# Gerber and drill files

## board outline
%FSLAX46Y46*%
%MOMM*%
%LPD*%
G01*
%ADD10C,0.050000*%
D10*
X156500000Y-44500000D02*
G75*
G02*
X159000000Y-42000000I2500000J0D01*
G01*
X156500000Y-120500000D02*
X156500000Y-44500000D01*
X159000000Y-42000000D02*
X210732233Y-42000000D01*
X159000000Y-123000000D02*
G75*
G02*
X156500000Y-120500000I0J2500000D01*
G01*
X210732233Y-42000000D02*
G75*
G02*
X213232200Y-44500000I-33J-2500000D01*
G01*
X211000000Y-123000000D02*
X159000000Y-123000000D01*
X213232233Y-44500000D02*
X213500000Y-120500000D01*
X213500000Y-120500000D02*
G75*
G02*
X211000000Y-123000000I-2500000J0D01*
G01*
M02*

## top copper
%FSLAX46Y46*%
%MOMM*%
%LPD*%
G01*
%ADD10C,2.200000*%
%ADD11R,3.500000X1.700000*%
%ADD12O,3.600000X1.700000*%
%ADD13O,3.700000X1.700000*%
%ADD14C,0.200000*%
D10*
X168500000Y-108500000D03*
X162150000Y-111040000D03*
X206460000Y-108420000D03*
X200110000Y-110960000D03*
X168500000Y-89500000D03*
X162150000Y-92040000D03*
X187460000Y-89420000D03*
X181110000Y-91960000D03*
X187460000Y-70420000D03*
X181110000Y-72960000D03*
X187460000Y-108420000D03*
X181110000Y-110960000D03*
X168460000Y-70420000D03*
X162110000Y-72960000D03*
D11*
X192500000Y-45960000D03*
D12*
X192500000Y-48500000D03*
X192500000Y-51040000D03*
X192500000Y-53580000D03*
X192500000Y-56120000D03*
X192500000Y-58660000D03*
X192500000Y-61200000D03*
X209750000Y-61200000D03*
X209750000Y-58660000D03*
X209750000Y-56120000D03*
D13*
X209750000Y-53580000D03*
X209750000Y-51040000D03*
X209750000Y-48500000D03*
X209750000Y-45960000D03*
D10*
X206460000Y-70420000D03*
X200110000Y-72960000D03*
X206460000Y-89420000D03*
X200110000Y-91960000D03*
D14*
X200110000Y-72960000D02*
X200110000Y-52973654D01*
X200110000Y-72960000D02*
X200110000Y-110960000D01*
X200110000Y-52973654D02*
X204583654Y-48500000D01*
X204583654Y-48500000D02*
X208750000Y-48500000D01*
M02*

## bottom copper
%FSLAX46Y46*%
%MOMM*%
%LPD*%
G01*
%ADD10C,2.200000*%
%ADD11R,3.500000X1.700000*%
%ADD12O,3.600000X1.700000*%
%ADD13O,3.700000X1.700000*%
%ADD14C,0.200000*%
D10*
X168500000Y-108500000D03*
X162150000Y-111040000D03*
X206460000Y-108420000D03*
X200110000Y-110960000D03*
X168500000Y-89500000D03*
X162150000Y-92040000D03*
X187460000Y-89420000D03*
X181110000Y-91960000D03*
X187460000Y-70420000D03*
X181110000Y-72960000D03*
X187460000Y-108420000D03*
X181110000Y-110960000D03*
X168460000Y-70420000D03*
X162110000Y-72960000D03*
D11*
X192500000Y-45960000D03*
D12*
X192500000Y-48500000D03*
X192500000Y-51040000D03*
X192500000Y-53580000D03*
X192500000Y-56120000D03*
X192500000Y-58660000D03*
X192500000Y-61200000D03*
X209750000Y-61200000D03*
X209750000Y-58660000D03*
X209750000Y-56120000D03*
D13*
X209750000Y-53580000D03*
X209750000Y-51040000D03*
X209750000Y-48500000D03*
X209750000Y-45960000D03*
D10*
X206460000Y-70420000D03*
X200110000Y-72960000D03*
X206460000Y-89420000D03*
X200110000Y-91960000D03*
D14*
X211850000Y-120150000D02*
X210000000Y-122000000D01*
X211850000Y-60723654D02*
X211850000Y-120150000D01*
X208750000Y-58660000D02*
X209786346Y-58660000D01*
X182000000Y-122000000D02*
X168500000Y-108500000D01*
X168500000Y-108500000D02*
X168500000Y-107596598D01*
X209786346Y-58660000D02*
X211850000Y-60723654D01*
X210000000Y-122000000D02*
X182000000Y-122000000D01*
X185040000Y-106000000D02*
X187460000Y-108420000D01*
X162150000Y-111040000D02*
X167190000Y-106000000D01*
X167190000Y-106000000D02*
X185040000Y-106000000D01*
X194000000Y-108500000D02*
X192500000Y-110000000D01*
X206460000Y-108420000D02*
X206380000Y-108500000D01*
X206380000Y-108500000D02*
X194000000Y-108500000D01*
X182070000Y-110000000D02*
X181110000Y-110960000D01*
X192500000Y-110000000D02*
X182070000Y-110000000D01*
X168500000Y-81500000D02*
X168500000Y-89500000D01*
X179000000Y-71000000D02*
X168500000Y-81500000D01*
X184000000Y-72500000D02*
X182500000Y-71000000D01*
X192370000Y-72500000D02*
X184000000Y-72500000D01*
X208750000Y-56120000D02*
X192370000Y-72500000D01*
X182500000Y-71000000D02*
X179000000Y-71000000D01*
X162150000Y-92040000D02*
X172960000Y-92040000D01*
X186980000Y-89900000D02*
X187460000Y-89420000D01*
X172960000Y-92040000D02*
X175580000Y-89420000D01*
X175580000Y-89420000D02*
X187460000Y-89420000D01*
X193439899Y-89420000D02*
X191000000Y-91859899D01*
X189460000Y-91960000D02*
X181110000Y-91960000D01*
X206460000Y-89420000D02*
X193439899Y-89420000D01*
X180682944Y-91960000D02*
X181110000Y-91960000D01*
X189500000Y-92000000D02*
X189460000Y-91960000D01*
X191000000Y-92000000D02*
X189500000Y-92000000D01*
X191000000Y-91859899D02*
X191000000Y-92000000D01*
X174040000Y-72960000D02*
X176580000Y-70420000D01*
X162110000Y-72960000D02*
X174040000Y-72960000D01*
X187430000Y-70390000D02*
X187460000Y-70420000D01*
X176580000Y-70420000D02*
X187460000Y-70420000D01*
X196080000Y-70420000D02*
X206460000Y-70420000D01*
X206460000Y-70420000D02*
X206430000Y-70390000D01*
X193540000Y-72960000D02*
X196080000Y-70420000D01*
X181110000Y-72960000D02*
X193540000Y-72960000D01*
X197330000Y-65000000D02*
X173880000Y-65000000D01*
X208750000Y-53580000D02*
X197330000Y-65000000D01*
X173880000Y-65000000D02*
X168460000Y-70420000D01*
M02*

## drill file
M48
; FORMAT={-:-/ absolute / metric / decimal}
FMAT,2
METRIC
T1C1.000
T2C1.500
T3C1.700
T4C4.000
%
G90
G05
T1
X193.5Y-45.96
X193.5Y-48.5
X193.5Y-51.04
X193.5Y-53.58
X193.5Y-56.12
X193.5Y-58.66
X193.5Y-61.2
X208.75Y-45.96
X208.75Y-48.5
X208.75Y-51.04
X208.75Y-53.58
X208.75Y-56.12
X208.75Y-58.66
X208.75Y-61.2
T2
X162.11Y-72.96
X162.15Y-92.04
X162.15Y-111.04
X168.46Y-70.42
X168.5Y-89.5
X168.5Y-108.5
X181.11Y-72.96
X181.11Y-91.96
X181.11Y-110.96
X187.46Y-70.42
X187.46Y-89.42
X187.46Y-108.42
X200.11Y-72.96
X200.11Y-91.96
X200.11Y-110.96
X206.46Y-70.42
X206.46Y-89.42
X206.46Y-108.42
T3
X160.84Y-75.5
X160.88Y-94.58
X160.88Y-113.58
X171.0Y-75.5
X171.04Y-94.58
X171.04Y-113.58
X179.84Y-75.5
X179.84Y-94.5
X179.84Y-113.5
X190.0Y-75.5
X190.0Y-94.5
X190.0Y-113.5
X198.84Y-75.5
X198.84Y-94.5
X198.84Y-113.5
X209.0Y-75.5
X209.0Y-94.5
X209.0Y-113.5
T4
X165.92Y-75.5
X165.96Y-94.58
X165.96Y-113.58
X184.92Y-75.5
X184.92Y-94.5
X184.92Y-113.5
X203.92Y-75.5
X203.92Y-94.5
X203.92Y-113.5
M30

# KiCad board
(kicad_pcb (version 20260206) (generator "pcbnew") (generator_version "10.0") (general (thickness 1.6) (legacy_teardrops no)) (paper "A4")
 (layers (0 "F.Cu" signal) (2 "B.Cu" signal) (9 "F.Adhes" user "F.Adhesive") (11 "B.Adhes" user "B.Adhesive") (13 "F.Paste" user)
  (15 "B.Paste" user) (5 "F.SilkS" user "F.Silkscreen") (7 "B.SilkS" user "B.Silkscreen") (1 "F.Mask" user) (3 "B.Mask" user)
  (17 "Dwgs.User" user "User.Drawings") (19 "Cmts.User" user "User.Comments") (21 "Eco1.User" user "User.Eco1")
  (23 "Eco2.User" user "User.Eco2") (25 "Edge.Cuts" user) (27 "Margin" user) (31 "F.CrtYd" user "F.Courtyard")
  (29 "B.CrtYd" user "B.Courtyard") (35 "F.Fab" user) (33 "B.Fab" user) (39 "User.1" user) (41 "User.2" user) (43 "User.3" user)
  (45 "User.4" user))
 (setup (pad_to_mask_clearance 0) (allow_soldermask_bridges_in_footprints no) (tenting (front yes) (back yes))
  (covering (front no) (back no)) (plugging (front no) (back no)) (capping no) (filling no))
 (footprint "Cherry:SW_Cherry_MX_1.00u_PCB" (layer "F.Cu") (at 168.5 108.5)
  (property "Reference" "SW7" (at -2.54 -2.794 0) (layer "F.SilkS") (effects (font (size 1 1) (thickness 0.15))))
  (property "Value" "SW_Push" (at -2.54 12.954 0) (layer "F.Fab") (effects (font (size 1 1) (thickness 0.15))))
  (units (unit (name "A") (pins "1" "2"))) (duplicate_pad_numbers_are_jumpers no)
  (pad "" np_thru_hole circle (at -7.62 5.08) (size 1.7 1.7) (drill 1.7) (layers "*.Cu" "*.Mask"))
  (pad "" np_thru_hole circle (at -2.54 5.08) (size 4 4) (drill 4) (layers "*.Cu" "*.Mask"))
  (pad "" np_thru_hole circle (at 2.54 5.08) (size 1.7 1.7) (drill 1.7) (layers "*.Cu" "*.Mask"))
  (pad "1" thru_hole circle (at 0 0) (size 2.2 2.2) (drill 1.5) (layers "*.Cu" "*.Mask") (remove_unused_layers no)
   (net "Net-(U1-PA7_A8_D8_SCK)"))
  (pad "2" thru_hole circle (at -6.35 2.54) (size 2.2 2.2) (drill 1.5) (layers "*.Cu" "*.Mask") (remove_unused_layers no)
   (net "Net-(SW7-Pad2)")))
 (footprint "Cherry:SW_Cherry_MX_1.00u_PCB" (layer "F.Cu") (at 206.46 108.42)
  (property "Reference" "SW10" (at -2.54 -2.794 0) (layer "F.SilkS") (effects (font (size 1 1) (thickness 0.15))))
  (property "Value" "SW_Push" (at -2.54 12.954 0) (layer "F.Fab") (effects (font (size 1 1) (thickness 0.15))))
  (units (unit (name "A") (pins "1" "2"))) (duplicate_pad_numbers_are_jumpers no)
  (pad "" np_thru_hole circle (at -7.62 5.08) (size 1.7 1.7) (drill 1.7) (layers "*.Cu" "*.Mask"))
  (pad "" np_thru_hole circle (at -2.54 5.08) (size 4 4) (drill 4) (layers "*.Cu" "*.Mask"))
  (pad "" np_thru_hole circle (at 2.54 5.08) (size 1.7 1.7) (drill 1.7) (layers "*.Cu" "*.Mask"))
  (pad "1" thru_hole circle (at 0 0) (size 2.2 2.2) (drill 1.5) (layers "*.Cu" "*.Mask") (remove_unused_layers no) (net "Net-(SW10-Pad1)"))
  (pad "2" thru_hole circle (at -6.35 2.54) (size 2.2 2.2) (drill 1.5) (layers "*.Cu" "*.Mask") (remove_unused_layers no) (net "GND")))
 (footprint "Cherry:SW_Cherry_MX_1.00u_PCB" (layer "F.Cu") (at 168.5 89.5)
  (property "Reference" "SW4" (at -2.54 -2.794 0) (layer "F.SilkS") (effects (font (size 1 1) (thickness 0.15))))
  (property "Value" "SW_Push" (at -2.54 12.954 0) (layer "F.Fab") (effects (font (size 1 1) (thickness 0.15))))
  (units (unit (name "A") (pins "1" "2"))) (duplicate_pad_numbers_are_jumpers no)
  (pad "" np_thru_hole circle (at -7.62 5.08) (size 1.7 1.7) (drill 1.7) (layers "*.Cu" "*.Mask"))
  (pad "" np_thru_hole circle (at -2.54 5.08) (size 4 4) (drill 4) (layers "*.Cu" "*.Mask"))
  (pad "" np_thru_hole circle (at 2.54 5.08) (size 1.7 1.7) (drill 1.7) (layers "*.Cu" "*.Mask"))
  (pad "1" thru_hole circle (at 0 0) (size 2.2 2.2) (drill 1.5) (layers "*.Cu" "*.Mask") (remove_unused_layers no)
   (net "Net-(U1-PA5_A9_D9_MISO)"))
  (pad "2" thru_hole circle (at -6.35 2.54) (size 2.2 2.2) (drill 1.5) (layers "*.Cu" "*.Mask") (remove_unused_layers no)
   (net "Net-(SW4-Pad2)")))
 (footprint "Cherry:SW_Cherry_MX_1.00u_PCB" (layer "F.Cu") (at 187.46 89.42)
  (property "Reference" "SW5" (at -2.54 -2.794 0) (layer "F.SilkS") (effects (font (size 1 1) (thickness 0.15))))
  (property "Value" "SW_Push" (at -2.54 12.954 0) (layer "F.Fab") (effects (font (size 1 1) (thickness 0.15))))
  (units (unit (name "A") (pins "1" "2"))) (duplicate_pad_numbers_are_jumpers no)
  (pad "" np_thru_hole circle (at -7.62 5.08) (size 1.7 1.7) (drill 1.7) (layers "*.Cu" "*.Mask"))
  (pad "" np_thru_hole circle (at -2.54 5.08) (size 4 4) (drill 4) (layers "*.Cu" "*.Mask"))
  (pad "" np_thru_hole circle (at 2.54 5.08) (size 1.7 1.7) (drill 1.7) (layers "*.Cu" "*.Mask"))
  (pad "1" thru_hole circle (at 0 0) (size 2.2 2.2) (drill 1.5) (layers "*.Cu" "*.Mask") (remove_unused_layers no) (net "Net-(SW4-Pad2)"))
  (pad "2" thru_hole circle (at -6.35 2.54) (size 2.2 2.2) (drill 1.5) (layers "*.Cu" "*.Mask") (remove_unused_layers no)
   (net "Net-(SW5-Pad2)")))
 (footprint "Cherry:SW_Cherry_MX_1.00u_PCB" (layer "F.Cu") (at 187.46 70.42)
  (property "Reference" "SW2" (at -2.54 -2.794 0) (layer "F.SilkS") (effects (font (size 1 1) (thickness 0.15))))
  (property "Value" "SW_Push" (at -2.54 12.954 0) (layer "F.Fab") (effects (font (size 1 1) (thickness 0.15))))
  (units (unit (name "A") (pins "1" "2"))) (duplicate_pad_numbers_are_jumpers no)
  (pad "" np_thru_hole circle (at -7.62 5.08) (size 1.7 1.7) (drill 1.7) (layers "*.Cu" "*.Mask"))
  (pad "" np_thru_hole circle (at -2.54 5.08) (size 4 4) (drill 4) (layers "*.Cu" "*.Mask"))
  (pad "" np_thru_hole circle (at 2.54 5.08) (size 1.7 1.7) (drill 1.7) (layers "*.Cu" "*.Mask"))
  (pad "1" thru_hole circle (at 0 0) (size 2.2 2.2) (drill 1.5) (layers "*.Cu" "*.Mask") (remove_unused_layers no) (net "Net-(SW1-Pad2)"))
  (pad "2" thru_hole circle (at -6.35 2.54) (size 2.2 2.2) (drill 1.5) (layers "*.Cu" "*.Mask") (remove_unused_layers no)
   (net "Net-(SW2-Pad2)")))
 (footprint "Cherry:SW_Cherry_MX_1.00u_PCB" (layer "F.Cu") (at 187.46 108.42)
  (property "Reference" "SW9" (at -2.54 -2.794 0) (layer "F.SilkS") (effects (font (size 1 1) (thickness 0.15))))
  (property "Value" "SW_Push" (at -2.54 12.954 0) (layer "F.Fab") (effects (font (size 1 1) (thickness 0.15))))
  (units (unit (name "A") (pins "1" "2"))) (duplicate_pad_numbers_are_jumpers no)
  (pad "" np_thru_hole circle (at -7.62 5.08) (size 1.7 1.7) (drill 1.7) (layers "*.Cu" "*.Mask"))
  (pad "" np_thru_hole circle (at -2.54 5.08) (size 4 4) (drill 4) (layers "*.Cu" "*.Mask"))
  (pad "" np_thru_hole circle (at 2.54 5.08) (size 1.7 1.7) (drill 1.7) (layers "*.Cu" "*.Mask"))
  (pad "1" thru_hole circle (at 0 0) (size 2.2 2.2) (drill 1.5) (layers "*.Cu" "*.Mask") (remove_unused_layers no) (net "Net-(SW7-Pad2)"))
  (pad "2" thru_hole circle (at -6.35 2.54) (size 2.2 2.2) (drill 1.5) (layers "*.Cu" "*.Mask") (remove_unused_layers no)
   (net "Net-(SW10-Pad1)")))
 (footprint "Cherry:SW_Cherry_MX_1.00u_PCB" (layer "F.Cu") (at 168.46 70.42)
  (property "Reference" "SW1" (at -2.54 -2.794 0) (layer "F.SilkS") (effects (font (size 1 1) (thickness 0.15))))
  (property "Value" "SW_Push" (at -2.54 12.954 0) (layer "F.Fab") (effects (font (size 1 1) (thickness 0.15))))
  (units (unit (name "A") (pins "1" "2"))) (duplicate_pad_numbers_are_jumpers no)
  (pad "" np_thru_hole circle (at -7.62 5.08) (size 1.7 1.7) (drill 1.7) (layers "*.Cu" "*.Mask"))
  (pad "" np_thru_hole circle (at -2.54 5.08) (size 4 4) (drill 4) (layers "*.Cu" "*.Mask"))
  (pad "" np_thru_hole circle (at 2.54 5.08) (size 1.7 1.7) (drill 1.7) (layers "*.Cu" "*.Mask"))
  (pad "1" thru_hole circle (at 0 0) (size 2.2 2.2) (drill 1.5) (layers "*.Cu" "*.Mask") (remove_unused_layers no)
   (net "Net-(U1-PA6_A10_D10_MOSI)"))
  (pad "2" thru_hole circle (at -6.35 2.54) (size 2.2 2.2) (drill 1.5) (layers "*.Cu" "*.Mask") (remove_unused_layers no)
   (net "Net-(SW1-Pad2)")))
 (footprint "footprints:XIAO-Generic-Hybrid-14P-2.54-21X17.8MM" (layer "F.Cu") (at 201.125 53.58)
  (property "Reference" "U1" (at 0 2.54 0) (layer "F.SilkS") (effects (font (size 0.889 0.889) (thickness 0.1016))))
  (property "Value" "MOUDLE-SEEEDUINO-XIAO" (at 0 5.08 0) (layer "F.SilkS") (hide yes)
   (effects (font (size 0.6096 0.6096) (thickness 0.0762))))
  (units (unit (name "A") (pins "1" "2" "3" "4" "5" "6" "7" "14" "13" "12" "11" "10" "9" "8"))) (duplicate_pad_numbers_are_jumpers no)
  (pad "1" thru_hole rect (at -7.625 -7.62) (size 3.5 1.7) (drill 1 (offset -1 0)) (layers "*.Cu" "*.Mask") (remove_unused_layers no)
   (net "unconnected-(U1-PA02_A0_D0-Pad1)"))
  (pad "2" thru_hole oval (at -7.625 -5.08) (size 3.6 1.7) (drill 1 (offset -1 0)) (layers "*.Cu" "*.Mask") (remove_unused_layers no)
   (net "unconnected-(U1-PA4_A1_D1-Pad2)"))
  (pad "3" thru_hole oval (at -7.625 -2.54) (size 3.6 1.7) (drill 1 (offset -1 0)) (layers "*.Cu" "*.Mask") (remove_unused_layers no)
   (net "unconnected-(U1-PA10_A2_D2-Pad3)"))
  (pad "4" thru_hole oval (at -7.625 0) (size 3.6 1.7) (drill 1 (offset -1 0)) (layers "*.Cu" "*.Mask") (remove_unused_layers no)
   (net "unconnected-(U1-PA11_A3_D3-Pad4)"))
  (pad "5" thru_hole oval (at -7.625 2.54) (size 3.6 1.7) (drill 1 (offset -1 0)) (layers "*.Cu" "*.Mask") (remove_unused_layers no)
   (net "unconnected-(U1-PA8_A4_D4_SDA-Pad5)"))
  (pad "6" thru_hole oval (at -7.625 5.08 180) (size 3.6 1.7) (drill 1 (offset 1 0)) (layers "*.Cu" "*.Mask") (remove_unused_layers no)
   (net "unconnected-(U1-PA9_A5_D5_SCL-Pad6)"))
  (pad "7" thru_hole oval (at -7.625 7.62) (size 3.6 1.7) (drill 1 (offset -1 0)) (layers "*.Cu" "*.Mask") (remove_unused_layers no)
   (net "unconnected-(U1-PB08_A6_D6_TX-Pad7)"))
  (pad "8" thru_hole oval (at 7.625 7.62) (size 3.6 1.7) (drill 1 (offset 1 0)) (layers "*.Cu" "*.Mask") (remove_unused_layers no)
   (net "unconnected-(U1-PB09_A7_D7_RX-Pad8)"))
  (pad "9" thru_hole oval (at 7.625 5.08) (size 3.6 1.7) (drill 1 (offset 1 0)) (layers "*.Cu" "*.Mask") (remove_unused_layers no)
   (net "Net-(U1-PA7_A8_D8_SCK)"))
  (pad "10" thru_hole oval (at 7.625 2.54) (size 3.6 1.7) (drill 1 (offset 1 0)) (layers "*.Cu" "*.Mask") (remove_unused_layers no)
   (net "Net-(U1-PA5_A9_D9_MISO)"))
  (pad "11" thru_hole oval (at 7.625 0) (size 3.7 1.7) (drill 1 (offset 1 0)) (layers "*.Cu" "*.Mask") (remove_unused_layers no)
   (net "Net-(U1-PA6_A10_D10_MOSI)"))
  (pad "12" thru_hole oval (at 7.625 -2.54) (size 3.7 1.7) (drill 1 (offset 1 0)) (layers "*.Cu" "*.Mask") (remove_unused_layers no)
   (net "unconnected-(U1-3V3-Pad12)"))
  (pad "13" thru_hole oval (at 7.625 -5.08) (size 3.7 1.7) (drill 1 (offset 1 0)) (layers "*.Cu" "*.Mask") (remove_unused_layers no)
   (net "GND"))
  (pad "14" thru_hole oval (at 7.625 -7.62) (size 3.7 1.7) (drill 1 (offset 1 0)) (layers "*.Cu" "*.Mask") (remove_unused_layers no)
   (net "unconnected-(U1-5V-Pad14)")))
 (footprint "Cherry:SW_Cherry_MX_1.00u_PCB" (layer "F.Cu") (at 206.46 70.42)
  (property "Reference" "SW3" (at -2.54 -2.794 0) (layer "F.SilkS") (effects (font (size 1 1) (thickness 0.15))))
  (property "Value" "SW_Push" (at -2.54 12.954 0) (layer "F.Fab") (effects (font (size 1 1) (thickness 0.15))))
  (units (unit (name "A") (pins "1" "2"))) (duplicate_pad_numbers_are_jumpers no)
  (pad "" np_thru_hole circle (at -7.62 5.08) (size 1.7 1.7) (drill 1.7) (layers "*.Cu" "*.Mask"))
  (pad "" np_thru_hole circle (at -2.54 5.08) (size 4 4) (drill 4) (layers "*.Cu" "*.Mask"))
  (pad "" np_thru_hole circle (at 2.54 5.08) (size 1.7 1.7) (drill 1.7) (layers "*.Cu" "*.Mask"))
  (pad "1" thru_hole circle (at 0 0) (size 2.2 2.2) (drill 1.5) (layers "*.Cu" "*.Mask") (remove_unused_layers no) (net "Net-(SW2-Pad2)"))
  (pad "2" thru_hole circle (at -6.35 2.54) (size 2.2 2.2) (drill 1.5) (layers "*.Cu" "*.Mask") (remove_unused_layers no) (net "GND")))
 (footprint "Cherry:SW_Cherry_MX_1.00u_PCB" (layer "F.Cu") (at 206.46 89.42)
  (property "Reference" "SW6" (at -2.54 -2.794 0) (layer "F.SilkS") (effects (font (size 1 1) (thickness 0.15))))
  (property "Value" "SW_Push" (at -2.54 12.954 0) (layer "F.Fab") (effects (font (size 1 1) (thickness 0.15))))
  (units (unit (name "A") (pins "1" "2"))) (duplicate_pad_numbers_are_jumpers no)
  (pad "" np_thru_hole circle (at -7.62 5.08) (size 1.7 1.7) (drill 1.7) (layers "*.Cu" "*.Mask"))
  (pad "" np_thru_hole circle (at -2.54 5.08) (size 4 4) (drill 4) (layers "*.Cu" "*.Mask"))
  (pad "" np_thru_hole circle (at 2.54 5.08) (size 1.7 1.7) (drill 1.7) (layers "*.Cu" "*.Mask"))
  (pad "1" thru_hole circle (at 0 0) (size 2.2 2.2) (drill 1.5) (layers "*.Cu" "*.Mask") (remove_unused_layers no) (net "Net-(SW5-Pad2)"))
  (pad "2" thru_hole circle (at -6.35 2.54) (size 2.2 2.2) (drill 1.5) (layers "*.Cu" "*.Mask") (remove_unused_layers no) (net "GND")))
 (gr_arc (start 156.5 44.5) (mid 157.232233 42.732233) (end 159 42) (stroke (width 0.05) (type default)) (layer "Edge.Cuts"))
 (gr_line (start 156.5 120.5) (end 156.5 44.5) (stroke (width 0.05) (type default)) (layer "Edge.Cuts"))
 (gr_line (start 159 42) (end 210.732233 42) (stroke (width 0.05) (type default)) (layer "Edge.Cuts"))
 (gr_arc (start 159 123) (mid 157.232233 122.267767) (end 156.5 120.5) (stroke (width 0.05) (type default)) (layer "Edge.Cuts"))
 (gr_arc (start 210.732233 42) (mid 212.5 42.732233) (end 213.232233 44.5) (stroke (width 0.05) (type default)) (layer "Edge.Cuts"))
 (gr_line (start 211 123) (end 159 123) (stroke (width 0.05) (type default)) (layer "Edge.Cuts"))
 (gr_line (start 213.232233 44.5) (end 213.5 120.5) (stroke (width 0.05) (type default)) (layer "Edge.Cuts"))
 (gr_arc (start 213.5 120.5) (mid 212.767767 122.267767) (end 211 123) (stroke (width 0.05) (type default)) (layer "Edge.Cuts"))
 (segment (start 211.85 120.15) (end 210 122) (width 0.2) (layer "B.Cu") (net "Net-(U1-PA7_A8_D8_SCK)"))
 (segment (start 211.85 60.723654) (end 211.85 120.15) (width 0.2) (layer "B.Cu") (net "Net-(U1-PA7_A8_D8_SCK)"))
 (segment (start 208.75 58.66) (end 209.786346 58.66) (width 0.2) (layer "B.Cu") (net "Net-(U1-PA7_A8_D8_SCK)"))
 (segment (start 182 122) (end 168.5 108.5) (width 0.2) (layer "B.Cu") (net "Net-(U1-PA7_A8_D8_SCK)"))
 (segment (start 168.5 108.5) (end 168.5 107.596598) (width 0.2) (layer "B.Cu") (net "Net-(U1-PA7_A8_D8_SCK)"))
 (segment (start 209.786346 58.66) (end 211.85 60.723654) (width 0.2) (layer "B.Cu") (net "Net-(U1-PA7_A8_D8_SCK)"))
 (segment (start 210 122) (end 182 122) (width 0.2) (layer "B.Cu") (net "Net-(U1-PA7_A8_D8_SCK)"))
 (segment (start 185.04 106) (end 187.46 108.42) (width 0.2) (layer "B.Cu") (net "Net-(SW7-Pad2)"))
 (segment (start 162.15 111.04) (end 167.19 106) (width 0.2) (layer "B.Cu") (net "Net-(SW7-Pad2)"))
 (segment (start 167.19 106) (end 185.04 106) (width 0.2) (layer "B.Cu") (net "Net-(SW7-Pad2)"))
 (segment (start 194 108.5) (end 192.5 110) (width 0.2) (layer "B.Cu") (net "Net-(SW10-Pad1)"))
 (segment (start 206.46 108.42) (end 206.38 108.5) (width 0.2) (layer "B.Cu") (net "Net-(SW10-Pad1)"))
 (segment (start 206.38 108.5) (end 194 108.5) (width 0.2) (layer "B.Cu") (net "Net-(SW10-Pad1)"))
 (segment (start 182.07 110) (end 181.11 110.96) (width 0.2) (layer "B.Cu") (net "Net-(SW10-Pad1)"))
 (segment (start 192.5 110) (end 182.07 110) (width 0.2) (layer "B.Cu") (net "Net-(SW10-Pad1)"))
 (segment (start 200.11 72.96) (end 200.11 52.973654) (width 0.2) (layer "F.Cu") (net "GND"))
 (segment (start 200.11 72.96) (end 200.11 110.96) (width 0.2) (layer "F.Cu") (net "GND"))
 (segment (start 200.11 52.973654) (end 204.583654 48.5) (width 0.2) (layer "F.Cu") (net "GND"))
 (segment (start 204.583654 48.5) (end 208.75 48.5) (width 0.2) (layer "F.Cu") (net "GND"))
 (segment (start 168.5 81.5) (end 168.5 89.5) (width 0.2) (layer "B.Cu") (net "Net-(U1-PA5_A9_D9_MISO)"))
 (segment (start 179 71) (end 168.5 81.5) (width 0.2) (layer "B.Cu") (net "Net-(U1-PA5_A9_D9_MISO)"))
 (segment (start 184 72.5) (end 182.5 71) (width 0.2) (layer "B.Cu") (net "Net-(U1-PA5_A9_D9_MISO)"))
 (segment (start 192.37 72.5) (end 184 72.5) (width 0.2) (layer "B.Cu") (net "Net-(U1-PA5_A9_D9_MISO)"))
 (segment (start 208.75 56.12) (end 192.37 72.5) (width 0.2) (layer "B.Cu") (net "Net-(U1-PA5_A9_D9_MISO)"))
 (segment (start 182.5 71) (end 179 71) (width 0.2) (layer "B.Cu") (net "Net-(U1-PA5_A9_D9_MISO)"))
 (segment (start 162.15 92.04) (end 172.96 92.04) (width 0.2) (layer "B.Cu") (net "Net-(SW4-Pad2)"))
 (segment (start 186.98 89.9) (end 187.46 89.42) (width 0.2) (layer "B.Cu") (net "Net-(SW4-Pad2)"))
 (segment (start 172.96 92.04) (end 175.58 89.42) (width 0.2) (layer "B.Cu") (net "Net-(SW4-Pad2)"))
 (segment (start 175.58 89.42) (end 187.46 89.42) (width 0.2) (layer "B.Cu") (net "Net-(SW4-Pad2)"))
 (segment (start 193.439899 89.42) (end 191 91.859899) (width 0.2) (layer "B.Cu") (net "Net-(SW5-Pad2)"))
 (segment (start 189.46 91.96) (end 181.11 91.96) (width 0.2) (layer "B.Cu") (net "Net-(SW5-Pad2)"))
 (segment (start 206.46 89.42) (end 193.439899 89.42) (width 0.2) (layer "B.Cu") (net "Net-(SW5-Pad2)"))
 (segment (start 180.682944 91.96) (end 181.11 91.96) (width 0.2) (layer "B.Cu") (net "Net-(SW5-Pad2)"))
 (segment (start 189.5 92) (end 189.46 91.96) (width 0.2) (layer "B.Cu") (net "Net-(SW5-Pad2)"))
 (segment (start 191 92) (end 189.5 92) (width 0.2) (layer "B.Cu") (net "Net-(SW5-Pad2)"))
 (segment (start 191 91.859899) (end 191 92) (width 0.2) (layer "B.Cu") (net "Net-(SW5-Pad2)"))
 (segment (start 174.04 72.96) (end 176.58 70.42) (width 0.2) (layer "B.Cu") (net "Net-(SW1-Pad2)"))
 (segment (start 162.11 72.96) (end 174.04 72.96) (width 0.2) (layer "B.Cu") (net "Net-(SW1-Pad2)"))
 (segment (start 187.43 70.39) (end 187.46 70.42) (width 0.2) (layer "B.Cu") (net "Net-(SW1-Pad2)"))
 (segment (start 176.58 70.42) (end 187.46 70.42) (width 0.2) (layer "B.Cu") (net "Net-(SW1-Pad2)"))
 (segment (start 196.08 70.42) (end 206.46 70.42) (width 0.2) (layer "B.Cu") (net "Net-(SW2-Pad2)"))
 (segment (start 206.46 70.42) (end 206.43 70.39) (width 0.2) (layer "B.Cu") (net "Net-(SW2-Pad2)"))
 (segment (start 193.54 72.96) (end 196.08 70.42) (width 0.2) (layer "B.Cu") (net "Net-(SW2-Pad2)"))
 (segment (start 181.11 72.96) (end 193.54 72.96) (width 0.2) (layer "B.Cu") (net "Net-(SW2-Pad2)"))
 (segment (start 197.33 65) (end 173.88 65) (width 0.2) (layer "B.Cu") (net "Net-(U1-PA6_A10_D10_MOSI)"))
 (segment (start 208.75 53.58) (end 197.33 65) (width 0.2) (layer "B.Cu") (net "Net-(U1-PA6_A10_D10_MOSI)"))
 (segment (start 173.88 65) (end 168.46 70.42) (width 0.2) (layer "B.Cu") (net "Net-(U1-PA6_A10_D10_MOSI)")))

